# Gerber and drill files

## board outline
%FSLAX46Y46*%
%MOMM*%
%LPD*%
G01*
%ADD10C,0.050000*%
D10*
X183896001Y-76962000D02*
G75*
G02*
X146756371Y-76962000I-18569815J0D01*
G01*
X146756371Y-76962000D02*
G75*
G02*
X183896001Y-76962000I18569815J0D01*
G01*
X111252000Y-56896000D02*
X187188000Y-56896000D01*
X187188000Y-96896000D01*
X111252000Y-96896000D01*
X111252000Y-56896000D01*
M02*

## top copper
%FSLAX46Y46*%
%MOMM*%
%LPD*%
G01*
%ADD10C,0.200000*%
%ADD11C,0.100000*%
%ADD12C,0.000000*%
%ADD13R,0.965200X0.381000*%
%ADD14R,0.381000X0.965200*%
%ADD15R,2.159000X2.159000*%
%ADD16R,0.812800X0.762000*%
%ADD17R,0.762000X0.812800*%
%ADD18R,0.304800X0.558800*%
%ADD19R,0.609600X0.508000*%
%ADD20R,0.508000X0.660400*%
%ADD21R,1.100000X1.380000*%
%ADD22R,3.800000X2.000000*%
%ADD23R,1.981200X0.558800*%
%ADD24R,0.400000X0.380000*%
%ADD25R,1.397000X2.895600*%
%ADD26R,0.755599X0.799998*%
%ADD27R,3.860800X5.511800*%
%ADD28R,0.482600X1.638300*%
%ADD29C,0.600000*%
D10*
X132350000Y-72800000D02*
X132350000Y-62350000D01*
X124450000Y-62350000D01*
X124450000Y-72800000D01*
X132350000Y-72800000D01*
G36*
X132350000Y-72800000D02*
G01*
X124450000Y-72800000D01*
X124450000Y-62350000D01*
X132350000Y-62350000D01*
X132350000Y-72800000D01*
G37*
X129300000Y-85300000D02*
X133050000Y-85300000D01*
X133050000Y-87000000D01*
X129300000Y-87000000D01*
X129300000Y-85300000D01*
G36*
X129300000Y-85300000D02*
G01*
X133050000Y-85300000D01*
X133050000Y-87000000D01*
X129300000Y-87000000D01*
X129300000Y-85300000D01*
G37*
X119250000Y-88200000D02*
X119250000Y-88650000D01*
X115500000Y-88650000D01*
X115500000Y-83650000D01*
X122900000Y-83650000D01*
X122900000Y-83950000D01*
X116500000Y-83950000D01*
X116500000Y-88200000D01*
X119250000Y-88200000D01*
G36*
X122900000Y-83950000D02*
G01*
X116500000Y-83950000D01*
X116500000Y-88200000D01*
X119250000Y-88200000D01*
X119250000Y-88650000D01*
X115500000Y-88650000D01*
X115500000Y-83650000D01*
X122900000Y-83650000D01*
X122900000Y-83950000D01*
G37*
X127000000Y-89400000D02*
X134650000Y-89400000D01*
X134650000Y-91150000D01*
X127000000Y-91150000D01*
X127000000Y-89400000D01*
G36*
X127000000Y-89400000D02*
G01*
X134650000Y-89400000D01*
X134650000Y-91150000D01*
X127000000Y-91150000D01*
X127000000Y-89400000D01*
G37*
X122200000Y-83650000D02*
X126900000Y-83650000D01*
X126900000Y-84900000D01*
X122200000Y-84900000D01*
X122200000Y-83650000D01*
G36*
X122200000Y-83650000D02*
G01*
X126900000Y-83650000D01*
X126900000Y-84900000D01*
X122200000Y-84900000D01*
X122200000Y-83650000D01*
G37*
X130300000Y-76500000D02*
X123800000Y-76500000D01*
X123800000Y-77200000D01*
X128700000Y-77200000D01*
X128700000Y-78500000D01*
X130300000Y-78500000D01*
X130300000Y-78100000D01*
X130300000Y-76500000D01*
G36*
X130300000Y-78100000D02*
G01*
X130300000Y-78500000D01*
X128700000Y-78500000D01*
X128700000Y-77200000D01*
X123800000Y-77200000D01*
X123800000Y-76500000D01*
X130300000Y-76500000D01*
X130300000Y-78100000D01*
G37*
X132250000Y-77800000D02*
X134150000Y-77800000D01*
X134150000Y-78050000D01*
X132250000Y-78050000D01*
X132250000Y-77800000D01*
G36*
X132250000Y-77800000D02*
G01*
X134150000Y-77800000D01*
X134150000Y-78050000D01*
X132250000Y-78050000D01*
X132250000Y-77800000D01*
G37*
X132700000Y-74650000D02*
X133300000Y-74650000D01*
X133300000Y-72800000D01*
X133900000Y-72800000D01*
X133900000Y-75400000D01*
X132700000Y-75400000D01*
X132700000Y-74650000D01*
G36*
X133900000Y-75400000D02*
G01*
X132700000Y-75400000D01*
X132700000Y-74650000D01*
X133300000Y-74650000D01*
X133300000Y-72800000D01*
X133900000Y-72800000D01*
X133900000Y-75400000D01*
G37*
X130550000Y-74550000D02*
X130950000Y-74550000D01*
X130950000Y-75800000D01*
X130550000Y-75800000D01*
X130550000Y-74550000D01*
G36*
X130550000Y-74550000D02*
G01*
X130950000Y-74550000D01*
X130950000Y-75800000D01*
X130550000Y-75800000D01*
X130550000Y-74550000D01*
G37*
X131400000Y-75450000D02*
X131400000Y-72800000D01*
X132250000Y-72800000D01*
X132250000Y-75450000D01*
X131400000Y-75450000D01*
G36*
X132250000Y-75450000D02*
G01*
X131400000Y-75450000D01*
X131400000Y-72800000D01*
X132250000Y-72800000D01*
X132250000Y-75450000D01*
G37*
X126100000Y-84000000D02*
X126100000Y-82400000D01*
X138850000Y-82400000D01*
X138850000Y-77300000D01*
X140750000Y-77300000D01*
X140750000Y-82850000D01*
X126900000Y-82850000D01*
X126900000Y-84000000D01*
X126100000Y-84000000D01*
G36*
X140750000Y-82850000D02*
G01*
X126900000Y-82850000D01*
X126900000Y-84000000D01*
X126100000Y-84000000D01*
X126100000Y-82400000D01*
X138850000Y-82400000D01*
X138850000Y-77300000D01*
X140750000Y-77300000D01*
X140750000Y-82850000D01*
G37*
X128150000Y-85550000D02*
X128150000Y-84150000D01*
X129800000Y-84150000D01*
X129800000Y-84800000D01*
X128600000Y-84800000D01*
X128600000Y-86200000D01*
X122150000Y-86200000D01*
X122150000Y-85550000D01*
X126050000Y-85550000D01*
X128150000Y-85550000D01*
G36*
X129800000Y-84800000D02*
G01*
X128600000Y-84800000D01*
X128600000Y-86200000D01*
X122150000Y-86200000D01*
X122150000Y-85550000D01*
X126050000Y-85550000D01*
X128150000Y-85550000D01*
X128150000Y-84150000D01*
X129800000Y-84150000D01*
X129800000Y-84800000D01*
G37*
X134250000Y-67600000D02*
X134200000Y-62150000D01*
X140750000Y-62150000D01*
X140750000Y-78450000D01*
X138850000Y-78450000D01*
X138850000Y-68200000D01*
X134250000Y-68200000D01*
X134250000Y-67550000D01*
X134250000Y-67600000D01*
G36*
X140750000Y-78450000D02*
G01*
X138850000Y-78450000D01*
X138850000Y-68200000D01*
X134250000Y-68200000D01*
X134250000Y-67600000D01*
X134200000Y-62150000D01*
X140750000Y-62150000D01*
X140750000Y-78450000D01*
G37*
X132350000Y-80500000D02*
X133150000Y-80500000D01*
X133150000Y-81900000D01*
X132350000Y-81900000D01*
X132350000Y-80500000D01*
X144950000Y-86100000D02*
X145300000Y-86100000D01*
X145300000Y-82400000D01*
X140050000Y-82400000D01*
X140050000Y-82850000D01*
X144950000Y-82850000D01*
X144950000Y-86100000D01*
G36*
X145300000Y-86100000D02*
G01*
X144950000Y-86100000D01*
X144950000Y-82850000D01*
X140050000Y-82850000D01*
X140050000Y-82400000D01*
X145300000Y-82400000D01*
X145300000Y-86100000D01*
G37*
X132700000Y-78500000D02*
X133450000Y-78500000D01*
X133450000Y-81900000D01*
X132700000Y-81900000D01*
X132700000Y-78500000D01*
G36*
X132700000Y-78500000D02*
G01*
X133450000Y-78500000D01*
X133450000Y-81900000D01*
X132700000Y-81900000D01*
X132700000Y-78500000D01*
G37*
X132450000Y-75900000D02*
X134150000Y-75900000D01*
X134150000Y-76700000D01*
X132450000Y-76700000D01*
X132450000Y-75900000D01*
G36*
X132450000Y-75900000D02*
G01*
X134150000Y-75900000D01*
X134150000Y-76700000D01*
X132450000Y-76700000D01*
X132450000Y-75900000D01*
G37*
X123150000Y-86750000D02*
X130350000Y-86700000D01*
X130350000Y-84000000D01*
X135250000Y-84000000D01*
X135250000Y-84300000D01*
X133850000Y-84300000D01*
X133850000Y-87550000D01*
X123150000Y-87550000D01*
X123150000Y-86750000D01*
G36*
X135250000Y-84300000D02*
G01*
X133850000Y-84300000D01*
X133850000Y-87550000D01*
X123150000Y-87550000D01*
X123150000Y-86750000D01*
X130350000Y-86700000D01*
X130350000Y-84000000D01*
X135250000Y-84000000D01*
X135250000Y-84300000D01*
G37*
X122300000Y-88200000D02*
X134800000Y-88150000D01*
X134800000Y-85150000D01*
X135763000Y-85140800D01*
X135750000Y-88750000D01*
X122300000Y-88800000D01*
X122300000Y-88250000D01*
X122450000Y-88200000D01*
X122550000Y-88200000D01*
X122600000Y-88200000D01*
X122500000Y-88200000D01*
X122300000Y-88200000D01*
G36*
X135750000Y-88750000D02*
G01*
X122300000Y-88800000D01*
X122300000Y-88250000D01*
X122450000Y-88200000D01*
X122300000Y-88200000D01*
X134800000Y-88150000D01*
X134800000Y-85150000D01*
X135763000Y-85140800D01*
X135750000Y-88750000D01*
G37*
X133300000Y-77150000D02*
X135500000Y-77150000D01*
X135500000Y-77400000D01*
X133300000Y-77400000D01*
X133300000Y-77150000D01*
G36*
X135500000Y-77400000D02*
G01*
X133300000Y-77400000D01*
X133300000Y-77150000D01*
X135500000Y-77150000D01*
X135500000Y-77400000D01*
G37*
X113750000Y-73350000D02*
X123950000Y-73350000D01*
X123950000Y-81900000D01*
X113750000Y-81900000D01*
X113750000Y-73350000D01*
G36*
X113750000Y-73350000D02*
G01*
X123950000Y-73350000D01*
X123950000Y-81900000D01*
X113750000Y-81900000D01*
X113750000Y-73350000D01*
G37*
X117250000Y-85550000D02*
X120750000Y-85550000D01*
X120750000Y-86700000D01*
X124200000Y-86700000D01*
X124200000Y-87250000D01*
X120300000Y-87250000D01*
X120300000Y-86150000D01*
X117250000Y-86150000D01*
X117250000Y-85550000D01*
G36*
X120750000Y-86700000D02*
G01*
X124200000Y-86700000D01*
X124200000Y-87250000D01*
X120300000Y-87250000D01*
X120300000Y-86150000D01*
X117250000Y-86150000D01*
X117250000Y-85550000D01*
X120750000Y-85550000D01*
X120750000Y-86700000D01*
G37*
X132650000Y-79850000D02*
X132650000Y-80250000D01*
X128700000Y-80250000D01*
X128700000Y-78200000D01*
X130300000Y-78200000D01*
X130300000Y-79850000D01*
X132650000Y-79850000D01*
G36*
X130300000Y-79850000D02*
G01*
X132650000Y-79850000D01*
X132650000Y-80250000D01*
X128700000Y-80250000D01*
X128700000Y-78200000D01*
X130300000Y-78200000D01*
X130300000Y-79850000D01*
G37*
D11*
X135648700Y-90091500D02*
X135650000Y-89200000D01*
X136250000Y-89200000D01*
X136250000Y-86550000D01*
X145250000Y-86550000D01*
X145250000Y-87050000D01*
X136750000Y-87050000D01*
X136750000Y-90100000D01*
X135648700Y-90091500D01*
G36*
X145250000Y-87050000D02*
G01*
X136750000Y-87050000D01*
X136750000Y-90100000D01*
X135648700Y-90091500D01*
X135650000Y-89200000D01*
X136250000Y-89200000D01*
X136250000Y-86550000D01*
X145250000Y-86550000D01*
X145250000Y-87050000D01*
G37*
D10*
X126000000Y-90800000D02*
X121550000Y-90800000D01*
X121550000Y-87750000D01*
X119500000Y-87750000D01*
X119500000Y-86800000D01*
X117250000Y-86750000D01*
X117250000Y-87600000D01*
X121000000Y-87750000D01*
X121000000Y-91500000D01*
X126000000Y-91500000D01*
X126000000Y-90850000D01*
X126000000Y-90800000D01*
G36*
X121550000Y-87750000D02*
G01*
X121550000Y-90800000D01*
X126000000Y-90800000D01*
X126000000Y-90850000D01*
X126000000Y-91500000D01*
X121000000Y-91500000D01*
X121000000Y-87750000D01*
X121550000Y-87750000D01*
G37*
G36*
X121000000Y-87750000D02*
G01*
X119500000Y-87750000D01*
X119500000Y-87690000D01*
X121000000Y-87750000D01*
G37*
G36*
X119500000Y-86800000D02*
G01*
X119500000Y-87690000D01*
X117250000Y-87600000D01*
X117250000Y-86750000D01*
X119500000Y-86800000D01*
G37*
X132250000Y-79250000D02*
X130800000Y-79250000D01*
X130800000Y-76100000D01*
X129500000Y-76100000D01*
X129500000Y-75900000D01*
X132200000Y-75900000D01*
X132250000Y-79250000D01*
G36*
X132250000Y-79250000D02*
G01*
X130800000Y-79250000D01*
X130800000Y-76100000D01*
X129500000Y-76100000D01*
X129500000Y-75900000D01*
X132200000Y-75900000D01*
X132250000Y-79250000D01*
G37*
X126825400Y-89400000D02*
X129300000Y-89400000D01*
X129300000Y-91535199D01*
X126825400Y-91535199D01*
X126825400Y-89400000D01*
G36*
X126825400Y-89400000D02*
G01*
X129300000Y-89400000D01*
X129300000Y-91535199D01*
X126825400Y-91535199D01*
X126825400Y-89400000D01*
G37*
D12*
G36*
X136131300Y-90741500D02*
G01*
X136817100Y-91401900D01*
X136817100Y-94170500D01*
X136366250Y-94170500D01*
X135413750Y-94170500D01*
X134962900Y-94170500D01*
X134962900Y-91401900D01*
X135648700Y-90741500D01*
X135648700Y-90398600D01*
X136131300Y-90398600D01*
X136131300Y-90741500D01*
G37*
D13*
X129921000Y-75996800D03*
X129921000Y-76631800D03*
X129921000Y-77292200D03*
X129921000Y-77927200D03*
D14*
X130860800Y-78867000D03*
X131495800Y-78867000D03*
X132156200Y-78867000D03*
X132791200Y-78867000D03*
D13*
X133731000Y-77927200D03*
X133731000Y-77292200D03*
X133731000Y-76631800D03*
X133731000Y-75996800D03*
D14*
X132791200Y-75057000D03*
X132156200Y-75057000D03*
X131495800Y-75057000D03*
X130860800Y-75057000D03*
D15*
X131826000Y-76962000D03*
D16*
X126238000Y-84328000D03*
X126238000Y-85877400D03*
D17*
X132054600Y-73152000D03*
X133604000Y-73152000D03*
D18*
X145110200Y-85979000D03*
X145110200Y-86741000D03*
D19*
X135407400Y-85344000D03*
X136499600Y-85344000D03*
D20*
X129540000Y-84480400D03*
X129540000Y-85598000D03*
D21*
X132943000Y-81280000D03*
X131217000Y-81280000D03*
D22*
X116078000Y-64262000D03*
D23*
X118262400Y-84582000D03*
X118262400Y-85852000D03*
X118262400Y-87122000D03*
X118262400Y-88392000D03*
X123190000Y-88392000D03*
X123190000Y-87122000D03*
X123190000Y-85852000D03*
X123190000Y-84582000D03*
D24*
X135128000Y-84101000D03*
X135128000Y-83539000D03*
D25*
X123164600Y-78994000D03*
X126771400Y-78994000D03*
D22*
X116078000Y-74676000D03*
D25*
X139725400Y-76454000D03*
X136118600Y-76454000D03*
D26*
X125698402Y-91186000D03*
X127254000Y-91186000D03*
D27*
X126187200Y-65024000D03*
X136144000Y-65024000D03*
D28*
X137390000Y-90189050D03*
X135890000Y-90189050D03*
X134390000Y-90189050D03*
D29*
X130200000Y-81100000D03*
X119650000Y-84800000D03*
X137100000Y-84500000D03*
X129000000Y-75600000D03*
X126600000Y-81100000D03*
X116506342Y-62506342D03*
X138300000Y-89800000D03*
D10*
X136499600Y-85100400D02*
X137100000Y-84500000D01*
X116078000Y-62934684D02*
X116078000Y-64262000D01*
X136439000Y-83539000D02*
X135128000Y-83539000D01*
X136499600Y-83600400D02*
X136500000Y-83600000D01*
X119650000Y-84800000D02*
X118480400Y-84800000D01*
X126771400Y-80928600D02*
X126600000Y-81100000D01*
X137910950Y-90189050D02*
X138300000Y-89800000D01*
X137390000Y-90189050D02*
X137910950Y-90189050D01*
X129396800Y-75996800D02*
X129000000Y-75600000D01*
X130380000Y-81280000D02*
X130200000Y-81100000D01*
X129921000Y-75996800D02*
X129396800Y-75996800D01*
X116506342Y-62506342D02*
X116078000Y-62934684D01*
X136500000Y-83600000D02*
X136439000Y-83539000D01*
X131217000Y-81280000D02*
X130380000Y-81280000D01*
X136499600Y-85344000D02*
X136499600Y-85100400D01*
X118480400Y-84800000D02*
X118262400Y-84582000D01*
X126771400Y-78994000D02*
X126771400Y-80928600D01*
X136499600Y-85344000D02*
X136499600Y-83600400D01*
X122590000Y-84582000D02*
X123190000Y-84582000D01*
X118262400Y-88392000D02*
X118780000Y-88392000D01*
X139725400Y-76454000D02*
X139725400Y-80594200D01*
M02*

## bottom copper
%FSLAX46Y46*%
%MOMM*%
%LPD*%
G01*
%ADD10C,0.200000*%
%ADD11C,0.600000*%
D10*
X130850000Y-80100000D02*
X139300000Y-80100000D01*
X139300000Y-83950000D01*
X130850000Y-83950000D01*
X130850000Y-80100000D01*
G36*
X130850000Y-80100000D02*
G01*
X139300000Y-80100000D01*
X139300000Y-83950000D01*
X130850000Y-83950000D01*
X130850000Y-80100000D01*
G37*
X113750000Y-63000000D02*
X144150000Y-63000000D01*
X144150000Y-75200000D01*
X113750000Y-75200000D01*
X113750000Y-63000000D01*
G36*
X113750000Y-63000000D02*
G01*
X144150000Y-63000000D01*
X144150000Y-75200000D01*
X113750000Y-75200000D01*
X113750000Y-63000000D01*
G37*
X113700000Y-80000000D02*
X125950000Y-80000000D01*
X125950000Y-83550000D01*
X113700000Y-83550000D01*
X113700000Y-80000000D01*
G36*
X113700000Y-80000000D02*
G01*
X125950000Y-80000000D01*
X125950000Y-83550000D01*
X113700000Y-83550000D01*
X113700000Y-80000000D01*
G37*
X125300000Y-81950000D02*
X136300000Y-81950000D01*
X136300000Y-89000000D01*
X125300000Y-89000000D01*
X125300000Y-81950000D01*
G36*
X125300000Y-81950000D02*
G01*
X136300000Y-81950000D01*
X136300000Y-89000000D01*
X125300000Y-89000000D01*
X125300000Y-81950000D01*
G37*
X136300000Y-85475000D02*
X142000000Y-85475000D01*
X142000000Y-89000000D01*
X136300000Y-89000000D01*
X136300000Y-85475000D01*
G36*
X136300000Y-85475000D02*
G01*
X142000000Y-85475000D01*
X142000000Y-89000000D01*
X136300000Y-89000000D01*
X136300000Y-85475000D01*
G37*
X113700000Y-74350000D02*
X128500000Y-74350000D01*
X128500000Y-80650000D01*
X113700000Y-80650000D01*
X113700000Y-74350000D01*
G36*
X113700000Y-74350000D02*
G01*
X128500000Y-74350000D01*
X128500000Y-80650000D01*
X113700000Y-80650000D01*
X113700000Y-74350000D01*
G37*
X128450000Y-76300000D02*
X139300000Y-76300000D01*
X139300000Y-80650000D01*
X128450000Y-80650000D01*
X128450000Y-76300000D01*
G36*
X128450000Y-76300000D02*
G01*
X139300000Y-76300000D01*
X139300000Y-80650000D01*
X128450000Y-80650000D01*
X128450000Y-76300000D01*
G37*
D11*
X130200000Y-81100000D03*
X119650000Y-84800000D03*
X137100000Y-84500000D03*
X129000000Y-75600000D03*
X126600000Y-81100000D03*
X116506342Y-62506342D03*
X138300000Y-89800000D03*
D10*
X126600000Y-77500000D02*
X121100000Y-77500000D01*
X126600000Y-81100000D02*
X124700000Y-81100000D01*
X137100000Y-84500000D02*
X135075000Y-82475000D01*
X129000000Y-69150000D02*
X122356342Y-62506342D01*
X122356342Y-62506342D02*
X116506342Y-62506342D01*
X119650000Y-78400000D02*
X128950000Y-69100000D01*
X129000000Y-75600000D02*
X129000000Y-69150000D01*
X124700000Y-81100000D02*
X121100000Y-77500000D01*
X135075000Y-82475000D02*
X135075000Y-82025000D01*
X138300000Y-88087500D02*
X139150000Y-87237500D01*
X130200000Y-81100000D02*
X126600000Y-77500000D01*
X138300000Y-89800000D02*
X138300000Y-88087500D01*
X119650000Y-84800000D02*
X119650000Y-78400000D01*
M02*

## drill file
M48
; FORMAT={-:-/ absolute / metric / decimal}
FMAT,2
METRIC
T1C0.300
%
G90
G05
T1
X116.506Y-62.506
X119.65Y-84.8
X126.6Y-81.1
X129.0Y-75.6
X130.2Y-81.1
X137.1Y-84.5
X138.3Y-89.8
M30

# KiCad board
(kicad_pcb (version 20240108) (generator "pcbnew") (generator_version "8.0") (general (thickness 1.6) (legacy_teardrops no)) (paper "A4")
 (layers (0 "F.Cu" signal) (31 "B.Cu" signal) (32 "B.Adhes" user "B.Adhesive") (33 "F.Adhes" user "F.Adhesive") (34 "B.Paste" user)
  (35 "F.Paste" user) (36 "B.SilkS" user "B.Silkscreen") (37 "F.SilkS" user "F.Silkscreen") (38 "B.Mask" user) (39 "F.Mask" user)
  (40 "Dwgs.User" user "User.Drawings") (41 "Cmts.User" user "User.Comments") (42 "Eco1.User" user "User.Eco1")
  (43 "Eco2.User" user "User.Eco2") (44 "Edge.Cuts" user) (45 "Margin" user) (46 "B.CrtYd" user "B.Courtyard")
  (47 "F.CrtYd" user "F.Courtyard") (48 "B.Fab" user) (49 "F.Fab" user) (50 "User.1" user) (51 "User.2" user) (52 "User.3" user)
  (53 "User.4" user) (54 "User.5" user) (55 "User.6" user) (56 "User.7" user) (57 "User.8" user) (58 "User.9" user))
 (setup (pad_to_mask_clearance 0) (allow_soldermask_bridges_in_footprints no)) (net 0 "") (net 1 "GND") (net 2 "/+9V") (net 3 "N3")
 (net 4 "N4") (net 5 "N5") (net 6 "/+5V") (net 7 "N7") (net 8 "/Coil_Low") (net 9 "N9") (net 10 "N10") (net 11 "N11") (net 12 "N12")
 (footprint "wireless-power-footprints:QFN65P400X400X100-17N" (layer "F.Cu") (at 131.826 76.962)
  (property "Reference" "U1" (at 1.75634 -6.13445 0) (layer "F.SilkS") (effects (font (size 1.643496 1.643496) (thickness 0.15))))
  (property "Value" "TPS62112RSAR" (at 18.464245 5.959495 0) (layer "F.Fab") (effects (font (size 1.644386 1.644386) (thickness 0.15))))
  (pad "1" smd rect (at -1.905 -0.9652 270) (size 0.381 0.9652) (layers "F.Cu" "F.Paste" "F.Mask") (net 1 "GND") (solder_mask_margin 0.102))
  (pad "2" smd rect (at -1.905 -0.3302 270) (size 0.381 0.9652) (layers "F.Cu" "F.Paste" "F.Mask") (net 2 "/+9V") (solder_mask_margin 0.102))
  (pad "3" smd rect (at -1.905 0.3302 270) (size 0.381 0.9652) (layers "F.Cu" "F.Paste" "F.Mask") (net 2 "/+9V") (solder_mask_margin 0.102))
  (pad "4" smd rect (at -1.905 0.9652 270) (size 0.381 0.9652) (layers "F.Cu" "F.Paste" "F.Mask") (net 2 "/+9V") (solder_mask_margin 0.102))
  (pad "5" smd rect (at -0.9652 1.905 180) (size 0.381 0.9652) (layers "F.Cu" "F.Paste" "F.Mask") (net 1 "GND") (solder_mask_margin 0.102))
  (pad "6" smd rect (at -0.3302 1.905 180) (size 0.381 0.9652) (layers "F.Cu" "F.Paste" "F.Mask") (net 1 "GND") (solder_mask_margin 0.102))
  (pad "7" smd rect (at 0.3302 1.905 180) (size 0.381 0.9652) (layers "F.Cu" "F.Paste" "F.Mask") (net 1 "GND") (solder_mask_margin 0.102))
  (pad "8" smd rect (at 0.9652 1.905 180) (size 0.381 0.9652) (layers "F.Cu" "F.Paste" "F.Mask") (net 2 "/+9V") (solder_mask_margin 0.102))
  (pad "9" smd rect (at 1.905 0.9652 270) (size 0.381 0.9652) (layers "F.Cu" "F.Paste" "F.Mask") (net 1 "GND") (solder_mask_margin 0.102))
  (pad "10" smd rect (at 1.905 0.3302 270) (size 0.381 0.9652) (layers "F.Cu" "F.Paste" "F.Mask") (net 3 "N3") (solder_mask_margin 0.102))
  (pad "11" smd rect (at 1.905 -0.3302 270) (size 0.381 0.9652) (layers "F.Cu" "F.Paste" "F.Mask") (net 1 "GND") (solder_mask_margin 0.102))
  (pad "12" smd rect (at 1.905 -0.9652 270) (size 0.381 0.9652) (layers "F.Cu" "F.Paste" "F.Mask") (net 1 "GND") (solder_mask_margin 0.102))
  (pad "13" smd rect (at 0.9652 -1.905 180) (size 0.381 0.9652) (layers "F.Cu" "F.Paste" "F.Mask") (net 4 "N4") (solder_mask_margin 0.102))
  (pad "14" smd rect (at 0.3302 -1.905 180) (size 0.381 0.9652) (layers "F.Cu" "F.Paste" "F.Mask") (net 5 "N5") (solder_mask_margin 0.102))
  (pad "15" smd rect (at -0.3302 -1.905 180) (size 0.381 0.9652) (layers "F.Cu" "F.Paste" "F.Mask") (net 5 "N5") (solder_mask_margin 0.102))
  (pad "16" smd rect (at -0.9652 -1.905 180) (size 0.381 0.9652) (layers "F.Cu" "F.Paste" "F.Mask") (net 1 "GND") (solder_mask_margin 0.102))
  (pad "17" smd rect (at 0 0) (size 2.159 2.159) (layers "F.Cu" "F.Paste" "F.Mask") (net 1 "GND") (solder_mask_margin 0.102)))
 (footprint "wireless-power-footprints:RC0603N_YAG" (layer "F.Cu") (at 126.238 85.1027 -90)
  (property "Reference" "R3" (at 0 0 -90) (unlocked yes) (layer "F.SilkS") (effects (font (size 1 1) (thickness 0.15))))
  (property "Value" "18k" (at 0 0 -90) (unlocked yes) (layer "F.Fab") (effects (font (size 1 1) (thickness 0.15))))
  (pad "1" smd rect (at -0.7747 0 270) (size 0.762 0.8128) (layers "F.Cu" "F.Paste" "F.Mask") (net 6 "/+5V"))
  (pad "2" smd rect (at 0.7747 0 270) (size 0.762 0.8128) (layers "F.Cu" "F.Paste" "F.Mask") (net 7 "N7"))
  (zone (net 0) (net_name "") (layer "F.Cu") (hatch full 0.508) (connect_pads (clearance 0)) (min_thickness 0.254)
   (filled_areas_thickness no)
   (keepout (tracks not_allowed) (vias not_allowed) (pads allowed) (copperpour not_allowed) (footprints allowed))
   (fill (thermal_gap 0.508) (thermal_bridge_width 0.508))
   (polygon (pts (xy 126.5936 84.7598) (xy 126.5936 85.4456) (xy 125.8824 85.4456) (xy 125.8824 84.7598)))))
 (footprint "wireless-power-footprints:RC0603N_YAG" (layer "F.Cu") (at 132.8293 73.152)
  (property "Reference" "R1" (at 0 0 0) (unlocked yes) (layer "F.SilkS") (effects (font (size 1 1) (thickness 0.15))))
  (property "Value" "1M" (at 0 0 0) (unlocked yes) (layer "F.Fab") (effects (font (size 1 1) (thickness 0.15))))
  (pad "1" smd rect (at -0.7747 0) (size 0.762 0.8128) (layers "F.Cu" "F.Paste" "F.Mask") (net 5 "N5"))
  (pad "2" smd rect (at 0.7747 0) (size 0.762 0.8128) (layers "F.Cu" "F.Paste" "F.Mask") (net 4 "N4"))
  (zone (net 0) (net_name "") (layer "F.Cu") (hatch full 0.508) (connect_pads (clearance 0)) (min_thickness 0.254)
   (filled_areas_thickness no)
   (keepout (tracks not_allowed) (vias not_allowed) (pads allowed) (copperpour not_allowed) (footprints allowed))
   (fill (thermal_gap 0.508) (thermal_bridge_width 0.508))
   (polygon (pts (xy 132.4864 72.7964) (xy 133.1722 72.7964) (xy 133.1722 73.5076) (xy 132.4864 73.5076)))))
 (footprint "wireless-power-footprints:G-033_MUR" (layer "F.Cu") (at 145.1102 86.36 -90)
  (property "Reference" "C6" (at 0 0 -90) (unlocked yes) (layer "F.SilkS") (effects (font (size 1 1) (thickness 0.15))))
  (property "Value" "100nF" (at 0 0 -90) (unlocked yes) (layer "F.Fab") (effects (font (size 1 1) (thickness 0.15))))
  (pad "1" smd rect (at -0.381 0 270) (size 0.5588 0.3048) (layers "F.Cu" "F.Paste" "F.Mask") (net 6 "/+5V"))
  (pad "2" smd rect (at 0.381 0 270) (size 0.5588 0.3048) (layers "F.Cu" "F.Paste" "F.Mask") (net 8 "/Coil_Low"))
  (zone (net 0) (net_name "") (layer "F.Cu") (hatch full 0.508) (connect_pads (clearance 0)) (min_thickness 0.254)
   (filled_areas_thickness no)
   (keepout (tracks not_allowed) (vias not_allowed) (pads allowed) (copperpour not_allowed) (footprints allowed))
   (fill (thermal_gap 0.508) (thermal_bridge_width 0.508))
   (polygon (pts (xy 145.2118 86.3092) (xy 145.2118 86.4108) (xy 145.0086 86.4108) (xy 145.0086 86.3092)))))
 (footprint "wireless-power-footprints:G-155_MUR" (layer "F.Cu") (at 135.9535 85.344)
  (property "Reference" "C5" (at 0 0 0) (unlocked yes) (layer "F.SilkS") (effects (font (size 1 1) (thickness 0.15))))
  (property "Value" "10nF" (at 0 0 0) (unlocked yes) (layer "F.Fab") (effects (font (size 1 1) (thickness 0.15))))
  (pad "1" smd rect (at -0.5461 0) (size 0.6096 0.508) (layers "F.Cu" "F.Paste" "F.Mask") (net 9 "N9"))
  (pad "2" smd rect (at 0.5461 0) (size 0.6096 0.508) (layers "F.Cu" "F.Paste" "F.Mask") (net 1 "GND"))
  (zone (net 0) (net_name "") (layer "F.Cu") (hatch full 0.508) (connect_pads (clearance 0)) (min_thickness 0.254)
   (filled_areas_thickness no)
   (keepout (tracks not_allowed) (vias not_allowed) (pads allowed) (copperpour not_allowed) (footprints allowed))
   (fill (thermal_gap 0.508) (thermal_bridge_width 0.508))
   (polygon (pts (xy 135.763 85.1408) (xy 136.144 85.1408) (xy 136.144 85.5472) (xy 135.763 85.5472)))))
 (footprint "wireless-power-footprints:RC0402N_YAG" (layer "F.Cu") (at 129.54 85.0392 -90)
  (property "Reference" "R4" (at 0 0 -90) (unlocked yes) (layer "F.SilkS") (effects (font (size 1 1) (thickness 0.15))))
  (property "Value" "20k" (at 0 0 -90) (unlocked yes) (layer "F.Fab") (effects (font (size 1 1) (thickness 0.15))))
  (pad "1" smd rect (at -0.5588 0 270) (size 0.6604 0.508) (layers "F.Cu" "F.Paste" "F.Mask") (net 7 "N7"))
  (pad "2" smd rect (at 0.5588 0 270) (size 0.6604 0.508) (layers "F.Cu" "F.Paste" "F.Mask") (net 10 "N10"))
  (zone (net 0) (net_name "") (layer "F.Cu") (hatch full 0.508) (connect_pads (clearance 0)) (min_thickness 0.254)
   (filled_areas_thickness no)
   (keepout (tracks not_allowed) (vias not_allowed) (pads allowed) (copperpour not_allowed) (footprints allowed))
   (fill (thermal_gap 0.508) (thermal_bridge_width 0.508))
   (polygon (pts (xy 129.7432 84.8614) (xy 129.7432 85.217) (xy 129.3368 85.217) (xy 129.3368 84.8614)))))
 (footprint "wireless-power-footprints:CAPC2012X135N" (layer "F.Cu") (at 132.08 81.28 180)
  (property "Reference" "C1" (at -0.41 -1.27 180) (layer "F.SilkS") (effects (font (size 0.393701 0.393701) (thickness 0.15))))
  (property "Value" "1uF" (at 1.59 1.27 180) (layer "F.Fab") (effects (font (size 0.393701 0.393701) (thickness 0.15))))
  (pad "1" smd rect (at -0.863 0 180) (size 1.1 1.38) (layers "F.Cu" "F.Paste" "F.Mask") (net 2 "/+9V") (solder_mask_margin 0.102))
  (pad "2" smd rect (at 0.863 0 180) (size 1.1 1.38) (layers "F.Cu" "F.Paste" "F.Mask") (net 1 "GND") (solder_mask_margin 0.102)))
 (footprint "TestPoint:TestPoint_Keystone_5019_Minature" (layer "F.Cu") (at 116.078 64.262)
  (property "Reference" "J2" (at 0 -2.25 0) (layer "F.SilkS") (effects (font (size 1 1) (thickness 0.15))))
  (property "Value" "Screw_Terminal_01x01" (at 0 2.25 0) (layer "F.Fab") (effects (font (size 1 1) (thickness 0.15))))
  (pad "1" smd rect (at 0 0) (size 3.8 2) (layers "F.Cu" "F.Paste" "F.Mask") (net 1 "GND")))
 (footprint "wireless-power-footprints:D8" (layer "F.Cu") (at 120.7262 86.487)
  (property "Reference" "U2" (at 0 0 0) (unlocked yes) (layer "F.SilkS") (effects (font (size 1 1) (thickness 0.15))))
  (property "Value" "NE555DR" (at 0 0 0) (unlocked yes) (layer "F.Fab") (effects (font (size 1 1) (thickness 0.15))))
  (pad "1" smd rect (at -2.4638 -1.905) (size 1.9812 0.5588) (layers "F.Cu" "F.Paste" "F.Mask") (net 1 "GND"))
  (pad "2" smd rect (at -2.4638 -0.635) (size 1.9812 0.5588) (layers "F.Cu" "F.Paste" "F.Mask") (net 10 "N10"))
  (pad "3" smd rect (at -2.4638 0.635) (size 1.9812 0.5588) (layers "F.Cu" "F.Paste" "F.Mask") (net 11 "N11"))
  (pad "4" smd rect (at -2.4638 1.905) (size 1.9812 0.5588) (layers "F.Cu" "F.Paste" "F.Mask") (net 6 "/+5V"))
  (pad "5" smd rect (at 2.4638 1.905) (size 1.9812 0.5588) (layers "F.Cu" "F.Paste" "F.Mask") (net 9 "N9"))
  (pad "6" smd rect (at 2.4638 0.635) (size 1.9812 0.5588) (layers "F.Cu" "F.Paste" "F.Mask") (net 10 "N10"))
  (pad "7" smd rect (at 2.4638 -0.635) (size 1.9812 0.5588) (layers "F.Cu" "F.Paste" "F.Mask") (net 7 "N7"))
  (pad "8" smd rect (at 2.4638 -1.905) (size 1.9812 0.5588) (layers "F.Cu" "F.Paste" "F.Mask") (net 6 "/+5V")))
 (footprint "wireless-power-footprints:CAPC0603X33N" (layer "F.Cu") (at 135.128 83.82 90)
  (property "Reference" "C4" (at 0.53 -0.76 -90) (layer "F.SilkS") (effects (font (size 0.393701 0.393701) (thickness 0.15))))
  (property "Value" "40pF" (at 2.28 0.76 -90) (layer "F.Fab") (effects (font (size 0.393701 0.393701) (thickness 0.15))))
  (pad "1" smd rect (at -0.281 0 90) (size 0.38 0.4) (layers "F.Cu" "F.Paste" "F.Mask") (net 10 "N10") (solder_mask_margin 0.102))
  (pad "2" smd rect (at 0.281 0 90) (size 0.38 0.4) (layers "F.Cu" "F.Paste" "F.Mask") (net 1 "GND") (solder_mask_margin 0.102)))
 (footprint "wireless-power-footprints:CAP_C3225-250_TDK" (layer "F.Cu") (at 124.968 78.994)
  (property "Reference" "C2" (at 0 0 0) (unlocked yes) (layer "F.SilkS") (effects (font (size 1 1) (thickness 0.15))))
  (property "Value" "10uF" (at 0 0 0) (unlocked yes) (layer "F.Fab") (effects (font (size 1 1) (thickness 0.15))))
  (pad "1" smd rect (at -1.8034 0) (size 1.397 2.8956) (layers "F.Cu" "F.Paste" "F.Mask") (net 2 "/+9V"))
  (pad "2" smd rect (at 1.8034 0) (size 1.397 2.8956) (layers "F.Cu" "F.Paste" "F.Mask") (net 1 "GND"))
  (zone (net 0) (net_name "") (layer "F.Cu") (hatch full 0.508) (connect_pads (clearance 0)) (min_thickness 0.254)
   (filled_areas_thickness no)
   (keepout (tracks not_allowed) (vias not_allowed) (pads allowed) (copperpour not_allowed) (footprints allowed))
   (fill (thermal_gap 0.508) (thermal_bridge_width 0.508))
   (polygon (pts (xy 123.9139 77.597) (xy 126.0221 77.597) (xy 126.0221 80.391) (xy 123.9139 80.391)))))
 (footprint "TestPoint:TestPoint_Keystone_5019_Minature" (layer "F.Cu") (at 116.078 74.676)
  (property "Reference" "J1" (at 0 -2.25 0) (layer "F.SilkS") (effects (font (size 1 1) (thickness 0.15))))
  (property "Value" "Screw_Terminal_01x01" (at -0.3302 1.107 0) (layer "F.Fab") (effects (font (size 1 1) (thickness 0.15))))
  (pad "1" smd rect (at 0 0) (size 3.8 2) (layers "F.Cu" "F.Paste" "F.Mask") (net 2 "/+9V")))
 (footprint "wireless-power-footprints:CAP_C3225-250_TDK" (layer "F.Cu") (at 137.922 76.454 180)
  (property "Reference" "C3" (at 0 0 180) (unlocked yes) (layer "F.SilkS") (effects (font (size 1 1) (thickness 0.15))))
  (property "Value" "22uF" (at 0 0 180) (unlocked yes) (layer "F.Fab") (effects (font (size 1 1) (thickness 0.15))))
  (pad "1" smd rect (at -1.8034 0 180) (size 1.397 2.8956) (layers "F.Cu" "F.Paste" "F.Mask") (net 6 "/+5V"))
  (pad "2" smd rect (at 1.8034 0 180) (size 1.397 2.8956) (layers "F.Cu" "F.Paste" "F.Mask") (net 3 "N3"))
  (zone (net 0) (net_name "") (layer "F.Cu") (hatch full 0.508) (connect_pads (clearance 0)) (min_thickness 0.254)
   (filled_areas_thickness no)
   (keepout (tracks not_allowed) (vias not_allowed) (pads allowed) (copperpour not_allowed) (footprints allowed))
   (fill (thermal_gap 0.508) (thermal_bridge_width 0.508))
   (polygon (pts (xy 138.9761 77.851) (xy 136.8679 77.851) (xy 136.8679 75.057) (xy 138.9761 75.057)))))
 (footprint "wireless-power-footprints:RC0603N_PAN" (layer "F.Cu") (at 126.476201 91.186)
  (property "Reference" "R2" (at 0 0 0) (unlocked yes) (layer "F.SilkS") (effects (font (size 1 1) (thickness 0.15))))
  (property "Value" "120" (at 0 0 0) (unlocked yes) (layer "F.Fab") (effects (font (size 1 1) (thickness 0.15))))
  (pad "1" smd rect (at -0.777799 0) (size 0.755599 0.799998) (layers "F.Cu" "F.Paste" "F.Mask") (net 11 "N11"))
  (pad "2" smd rect (at 0.777799 0) (size 0.755599 0.799998) (layers "F.Cu" "F.Paste" "F.Mask") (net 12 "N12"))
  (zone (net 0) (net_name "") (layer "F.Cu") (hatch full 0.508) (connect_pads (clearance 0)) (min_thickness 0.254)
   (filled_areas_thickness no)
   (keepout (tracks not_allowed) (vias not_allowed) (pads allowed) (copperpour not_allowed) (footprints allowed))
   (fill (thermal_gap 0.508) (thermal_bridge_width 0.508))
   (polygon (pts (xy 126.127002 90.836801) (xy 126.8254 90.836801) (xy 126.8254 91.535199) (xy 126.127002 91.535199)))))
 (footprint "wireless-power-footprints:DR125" (layer "F.Cu") (at 131.1656 65.024)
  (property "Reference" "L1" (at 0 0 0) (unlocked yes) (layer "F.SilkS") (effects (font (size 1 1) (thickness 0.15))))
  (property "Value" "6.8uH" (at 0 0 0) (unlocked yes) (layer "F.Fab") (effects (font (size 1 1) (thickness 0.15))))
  (pad "1" smd rect (at -4.9784 0) (size 3.8608 5.5118) (layers "F.Cu" "F.Paste" "F.Mask") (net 5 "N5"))
  (pad "2" smd rect (at 4.9784 0) (size 3.8608 5.5118) (layers "F.Cu" "F.Paste" "F.Mask") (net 6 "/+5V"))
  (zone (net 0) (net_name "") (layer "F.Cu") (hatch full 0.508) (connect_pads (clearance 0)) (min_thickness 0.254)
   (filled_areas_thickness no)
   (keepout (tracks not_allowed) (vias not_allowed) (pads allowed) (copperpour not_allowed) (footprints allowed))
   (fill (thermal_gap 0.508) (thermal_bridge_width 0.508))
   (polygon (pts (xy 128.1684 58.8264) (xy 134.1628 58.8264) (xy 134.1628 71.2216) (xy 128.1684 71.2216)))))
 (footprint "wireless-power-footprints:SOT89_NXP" (layer "F.Cu") (at 135.89 91.694 180)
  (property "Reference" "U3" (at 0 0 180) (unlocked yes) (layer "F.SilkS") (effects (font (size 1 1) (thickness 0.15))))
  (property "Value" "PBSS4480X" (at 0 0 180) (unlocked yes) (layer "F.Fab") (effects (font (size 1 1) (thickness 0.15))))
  (fp_poly
   (pts (xy -0.2413 1.2954) (xy -0.2413 0.9525) (xy -0.9271 0.2921) (xy -0.9271 -2.4765) (xy -0.47625 -2.4765) (xy 0.47625 -2.4765)
    (xy 0.9271 -2.4765) (xy 0.9271 0.2921) (xy 0.2413 0.9525) (xy 0.2413 1.2954))
   (stroke (width 0) (type solid)) (fill solid) (layer "F.Cu"))
  (pad "1" smd rect (at -1.5 1.50495 180) (size 0.4826 1.6383) (layers "F.Cu" "F.Paste" "F.Mask") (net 1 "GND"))
  (pad "2" smd rect (at 0 1.50495 180) (size 0.4826 1.6383) (layers "F.Cu" "F.Paste" "F.Mask") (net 8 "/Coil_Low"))
  (pad "3" smd rect (at 1.5 1.50495 180) (size 0.4826 1.6383) (layers "F.Cu" "F.Paste" "F.Mask") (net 12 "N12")))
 (gr_poly
  (pts (xy 132.35 72.8) (xy 132.35 62.35) (xy 124.45 62.35) (xy 124.45 72.8)) (stroke (width 0.2) (type solid)) (fill solid) (layer "F.Cu")
  (net 5))
 (gr_rect (start 129.3 85.3) (end 133.05 87) (stroke (width 0.2) (type solid)) (fill solid) (layer "F.Cu") (net 10))
 (gr_poly
  (pts (xy 119.25 88.2) (xy 119.25 88.65) (xy 115.5 88.65) (xy 115.5 83.65) (xy 122.9 83.65) (xy 122.9 83.95) (xy 116.5 83.95)
   (xy 116.5 88.2))
  (stroke (width 0.2) (type solid)) (fill solid) (layer "F.Cu") (net 6))
 (gr_rect (start 127 89.4) (end 134.65 91.15) (stroke (width 0.2) (type solid)) (fill solid) (layer "F.Cu") (net 12))
 (gr_rect (start 122.2 83.65) (end 126.9 84.9) (stroke (width 0.2) (type solid)) (fill solid) (layer "F.Cu") (net 6))
 (gr_poly
  (pts (xy 130.3 76.5) (xy 123.8 76.5) (xy 123.8 77.2) (xy 128.7 77.2) (xy 128.7 78.5) (xy 130.3 78.5) (xy 130.3 78.1))
  (stroke (width 0.2) (type solid)) (fill solid) (layer "F.Cu") (net 2))
 (gr_rect (start 132.25 77.8) (end 134.15 78.05) (stroke (width 0.2) (type solid)) (fill solid) (layer "F.Cu") (net 1))
 (gr_poly
  (pts (xy 132.7 74.65) (xy 133.3 74.65) (xy 133.3 72.8) (xy 133.9 72.8) (xy 133.9 75.4) (xy 132.7 75.4)) (stroke (width 0.2) (type solid))
  (fill solid) (layer "F.Cu") (net 4))
 (gr_rect (start 130.55 74.55) (end 130.95 75.8) (stroke (width 0.2) (type solid)) (fill solid) (layer "F.Cu") (net 1))
 (gr_poly
  (pts (xy 131.4 75.45) (xy 131.4 72.8) (xy 132.25 72.8) (xy 132.25 75.45)) (stroke (width 0.2) (type solid)) (fill solid) (layer "F.Cu")
  (net 5))
 (gr_poly
  (pts (xy 126.1 84) (xy 126.1 82.4) (xy 138.85 82.4) (xy 138.85 77.3) (xy 140.75 77.3) (xy 140.75 82.85) (xy 126.9 82.85) (xy 126.9 84))
  (stroke (width 0.2) (type solid)) (fill solid) (layer "F.Cu") (net 6))
 (gr_poly
  (pts (xy 128.15 85.55) (xy 128.15 84.15) (xy 129.8 84.15) (xy 129.8 84.8) (xy 128.6 84.8) (xy 128.6 86.2) (xy 122.15 86.2)
   (xy 122.15 85.55) (xy 126.05 85.55))
  (stroke (width 0.2) (type solid)) (fill solid) (layer "F.Cu") (net 7))
 (gr_poly
  (pts (xy 134.25 67.6) (xy 134.2 62.15) (xy 140.75 62.15) (xy 140.75 78.45) (xy 138.85 78.45) (xy 138.85 68.2) (xy 134.25 68.2)
   (xy 134.25 67.55))
  (stroke (width 0.2) (type solid)) (fill solid) (layer "F.Cu") (net 6))
 (gr_rect (start 132.35 80.5) (end 133.15 81.9) (stroke (width 0.2) (type default)) (fill none) (layer "F.Cu") (net 2))
 (gr_poly
  (pts (xy 144.95 86.1) (xy 145.3 86.1) (xy 145.3 82.4) (xy 140.05 82.4) (xy 140.05 82.85) (xy 144.95 82.85) (xy 144.95 86.1))
  (stroke (width 0.2) (type solid)) (fill solid) (layer "F.Cu") (net 6))
 (gr_rect (start 132.7 78.5) (end 133.45 81.9) (stroke (width 0.2) (type solid)) (fill solid) (layer "F.Cu") (net 2))
 (gr_rect (start 132.45 75.9) (end 134.15 76.7) (stroke (width 0.2) (type solid)) (fill solid) (layer "F.Cu") (net 1))
 (gr_poly
  (pts (xy 123.15 86.75) (xy 130.35 86.7) (xy 130.35 84) (xy 135.25 84) (xy 135.25 84.3) (xy 133.85 84.3) (xy 133.85 87.55)
   (xy 123.15 87.55))
  (stroke (width 0.2) (type solid)) (fill solid) (layer "F.Cu") (net 10))
 (gr_poly
  (pts (xy 122.3 88.2) (xy 134.8 88.15) (xy 134.8 85.15) (xy 135.763 85.1408) (xy 135.75 88.75) (xy 122.3 88.8) (xy 122.3 88.25)
   (xy 122.45 88.2) (xy 122.55 88.2) (xy 122.6 88.2) (xy 122.5 88.2))
  (stroke (width 0.2) (type solid)) (fill solid) (layer "F.Cu") (net 9))
 (gr_poly
  (pts (xy 133.3 77.15) (xy 135.5 77.15) (xy 135.5 77.4) (xy 133.3 77.4)) (stroke (width 0.2) (type solid)) (fill solid) (layer "F.Cu")
  (net 3))
 (gr_rect (start 113.75 73.35) (end 123.95 81.9) (stroke (width 0.2) (type solid)) (fill solid) (layer "F.Cu") (net 2))
 (gr_poly
  (pts (xy 117.25 85.55) (xy 120.75 85.55) (xy 120.75 86.7) (xy 124.2 86.7) (xy 124.2 87.25) (xy 120.3 87.25) (xy 120.3 86.15)
   (xy 117.25 86.15))
  (stroke (width 0.2) (type solid)) (fill solid) (layer "F.Cu") (net 10))
 (gr_poly
  (pts (xy 132.65 79.85) (xy 132.65 80.25) (xy 128.7 80.25) (xy 128.7 78.2) (xy 130.3 78.2) (xy 130.3 79.85))
  (stroke (width 0.2) (type solid)) (fill solid) (layer "F.Cu") (net 2))
 (gr_poly
  (pts (xy 135.6487 90.0915) (xy 135.65 89.2) (xy 136.25 89.2) (xy 136.25 86.55) (xy 145.25 86.55) (xy 145.25 87.05) (xy 136.75 87.05)
   (xy 136.75 90.1))
  (stroke (width 0.1) (type solid)) (fill solid) (layer "F.Cu") (net 8))
 (gr_poly
  (pts (xy 126 90.8) (xy 121.55 90.8) (xy 121.55 87.75) (xy 119.5 87.75) (xy 119.5 86.8) (xy 117.25 86.75) (xy 117.25 87.6) (xy 121 87.75)
   (xy 121 91.5) (xy 126 91.5) (xy 126 90.85))
  (stroke (width 0.2) (type solid)) (fill solid) (layer "F.Cu") (net 11))
 (gr_poly
  (pts (xy 132.25 79.25) (xy 130.8 79.25) (xy 130.8 76.1) (xy 129.5 76.1) (xy 129.5 75.9) (xy 132.2 75.9)) (stroke (width 0.2) (type solid))
  (fill solid) (layer "F.Cu") (net 1))
 (gr_rect (start 126.8254 89.4) (end 129.3 91.535199) (stroke (width 0.2) (type solid)) (fill solid) (layer "F.Cu") (net 12))
 (gr_rect (start 130.85 80.1) (end 139.3 83.95) (stroke (width 0.2) (type solid)) (fill solid) (layer "B.Cu") (net 1))
 (gr_rect (start 113.75 63) (end 144.15 75.2) (stroke (width 0.2) (type solid)) (fill solid) (layer "B.Cu") (net 1))
 (gr_rect (start 113.7 80) (end 125.95 83.55) (stroke (width 0.2) (type solid)) (fill solid) (layer "B.Cu") (net 1))
 (gr_rect (start 125.3 81.95) (end 136.3 89) (stroke (width 0.2) (type solid)) (fill solid) (layer "B.Cu") (net 1))
 (gr_rect (start 136.3 85.475) (end 142 89) (stroke (width 0.2) (type solid)) (fill solid) (layer "B.Cu") (net 1))
 (gr_rect (start 113.7 74.35) (end 128.5 80.65) (stroke (width 0.2) (type solid)) (fill solid) (layer "B.Cu") (net 1))
 (gr_rect (start 128.45 76.3) (end 139.3 80.65) (stroke (width 0.2) (type solid)) (fill solid) (layer "B.Cu") (net 1))
 (gr_circle (center 165.326186 76.962) (end 177.264186 91.186) (stroke (width 0.05) (type default)) (fill none) (layer "Edge.Cuts"))
 (gr_rect (start 111.252 56.896) (end 187.188 96.896) (stroke (width 0.05) (type default)) (fill none) (layer "Edge.Cuts"))
 (segment (start 136.4996 85.1004) (end 137.1 84.5) (width 0.2) (layer "F.Cu") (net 1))
 (segment (start 116.078 62.934684) (end 116.078 64.262) (width 0.2) (layer "F.Cu") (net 1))
 (segment (start 136.439 83.539) (end 135.128 83.539) (width 0.2) (layer "F.Cu") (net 1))
 (segment (start 136.4996 83.6004) (end 136.5 83.6) (width 0.2) (layer "F.Cu") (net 1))
 (segment (start 119.65 84.8) (end 118.4804 84.8) (width 0.2) (layer "F.Cu") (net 1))
 (segment (start 126.7714 80.9286) (end 126.6 81.1) (width 0.2) (layer "F.Cu") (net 1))
 (segment (start 137.91095 90.18905) (end 138.3 89.8) (width 0.2) (layer "F.Cu") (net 1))
 (segment (start 137.39 90.18905) (end 137.91095 90.18905) (width 0.2) (layer "F.Cu") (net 1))
 (segment (start 129.3968 75.9968) (end 129 75.6) (width 0.2) (layer "F.Cu") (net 1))
 (segment (start 130.38 81.28) (end 130.2 81.1) (width 0.2) (layer "F.Cu") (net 1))
 (segment (start 129.921 75.9968) (end 129.3968 75.9968) (width 0.2) (layer "F.Cu") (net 1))
 (segment (start 116.506342 62.506342) (end 116.078 62.934684) (width 0.2) (layer "F.Cu") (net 1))
 (segment (start 136.5 83.6) (end 136.439 83.539) (width 0.2) (layer "F.Cu") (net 1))
 (segment (start 131.217 81.28) (end 130.38 81.28) (width 0.2) (layer "F.Cu") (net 1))
 (segment (start 136.4996 85.344) (end 136.4996 85.1004) (width 0.2) (layer "F.Cu") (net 1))
 (segment (start 118.4804 84.8) (end 118.2624 84.582) (width 0.2) (layer "F.Cu") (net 1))
 (segment (start 126.7714 78.994) (end 126.7714 80.9286) (width 0.2) (layer "F.Cu") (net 1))
 (segment (start 136.4996 85.344) (end 136.4996 83.6004) (width 0.2) (layer "F.Cu") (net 1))
 (via (at 130.2 81.1) (size 0.6) (drill 0.3) (layers "F.Cu" "B.Cu") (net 1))
 (via (at 119.65 84.8) (size 0.6) (drill 0.3) (layers "F.Cu" "B.Cu") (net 1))
 (via (at 137.1 84.5) (size 0.6) (drill 0.3) (layers "F.Cu" "B.Cu") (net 1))
 (via (at 129 75.6) (size 0.6) (drill 0.3) (layers "F.Cu" "B.Cu") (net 1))
 (via (at 126.6 81.1) (size 0.6) (drill 0.3) (layers "F.Cu" "B.Cu") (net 1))
 (via (at 116.506342 62.506342) (size 0.6) (drill 0.3) (layers "F.Cu" "B.Cu") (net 1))
 (via (at 138.3 89.8) (size 0.6) (drill 0.3) (layers "F.Cu" "B.Cu") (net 1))
 (segment (start 126.6 77.5) (end 121.1 77.5) (width 0.2) (layer "B.Cu") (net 1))
 (segment (start 126.6 81.1) (end 124.7 81.1) (width 0.2) (layer "B.Cu") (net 1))
 (segment (start 137.1 84.5) (end 135.075 82.475) (width 0.2) (layer "B.Cu") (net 1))
 (segment (start 129 69.15) (end 122.356342 62.506342) (width 0.2) (layer "B.Cu") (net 1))
 (segment (start 122.356342 62.506342) (end 116.506342 62.506342) (width 0.2) (layer "B.Cu") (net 1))
 (segment (start 119.65 78.4) (end 128.95 69.1) (width 0.2) (layer "B.Cu") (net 1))
 (segment (start 129 75.6) (end 129 69.15) (width 0.2) (layer "B.Cu") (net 1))
 (segment (start 124.7 81.1) (end 121.1 77.5) (width 0.2) (layer "B.Cu") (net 1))
 (segment (start 135.075 82.475) (end 135.075 82.025) (width 0.2) (layer "B.Cu") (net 1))
 (segment (start 138.3 88.0875) (end 139.15 87.2375) (width 0.2) (layer "B.Cu") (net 1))
 (segment (start 130.2 81.1) (end 126.6 77.5) (width 0.2) (layer "B.Cu") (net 1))
 (segment (start 138.3 89.8) (end 138.3 88.0875) (width 0.2) (layer "B.Cu") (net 1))
 (segment (start 119.65 84.8) (end 119.65 78.4) (width 0.2) (layer "B.Cu") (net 1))
 (segment (start 122.59 84.582) (end 123.19 84.582) (width 0.2) (layer "F.Cu") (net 6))
 (segment (start 118.2624 88.392) (end 118.78 88.392) (width 0.2) (layer "F.Cu") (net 6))
 (segment (start 139.7254 76.454) (end 139.7254 80.5942) (width 0.2) (layer "F.Cu") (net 6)))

